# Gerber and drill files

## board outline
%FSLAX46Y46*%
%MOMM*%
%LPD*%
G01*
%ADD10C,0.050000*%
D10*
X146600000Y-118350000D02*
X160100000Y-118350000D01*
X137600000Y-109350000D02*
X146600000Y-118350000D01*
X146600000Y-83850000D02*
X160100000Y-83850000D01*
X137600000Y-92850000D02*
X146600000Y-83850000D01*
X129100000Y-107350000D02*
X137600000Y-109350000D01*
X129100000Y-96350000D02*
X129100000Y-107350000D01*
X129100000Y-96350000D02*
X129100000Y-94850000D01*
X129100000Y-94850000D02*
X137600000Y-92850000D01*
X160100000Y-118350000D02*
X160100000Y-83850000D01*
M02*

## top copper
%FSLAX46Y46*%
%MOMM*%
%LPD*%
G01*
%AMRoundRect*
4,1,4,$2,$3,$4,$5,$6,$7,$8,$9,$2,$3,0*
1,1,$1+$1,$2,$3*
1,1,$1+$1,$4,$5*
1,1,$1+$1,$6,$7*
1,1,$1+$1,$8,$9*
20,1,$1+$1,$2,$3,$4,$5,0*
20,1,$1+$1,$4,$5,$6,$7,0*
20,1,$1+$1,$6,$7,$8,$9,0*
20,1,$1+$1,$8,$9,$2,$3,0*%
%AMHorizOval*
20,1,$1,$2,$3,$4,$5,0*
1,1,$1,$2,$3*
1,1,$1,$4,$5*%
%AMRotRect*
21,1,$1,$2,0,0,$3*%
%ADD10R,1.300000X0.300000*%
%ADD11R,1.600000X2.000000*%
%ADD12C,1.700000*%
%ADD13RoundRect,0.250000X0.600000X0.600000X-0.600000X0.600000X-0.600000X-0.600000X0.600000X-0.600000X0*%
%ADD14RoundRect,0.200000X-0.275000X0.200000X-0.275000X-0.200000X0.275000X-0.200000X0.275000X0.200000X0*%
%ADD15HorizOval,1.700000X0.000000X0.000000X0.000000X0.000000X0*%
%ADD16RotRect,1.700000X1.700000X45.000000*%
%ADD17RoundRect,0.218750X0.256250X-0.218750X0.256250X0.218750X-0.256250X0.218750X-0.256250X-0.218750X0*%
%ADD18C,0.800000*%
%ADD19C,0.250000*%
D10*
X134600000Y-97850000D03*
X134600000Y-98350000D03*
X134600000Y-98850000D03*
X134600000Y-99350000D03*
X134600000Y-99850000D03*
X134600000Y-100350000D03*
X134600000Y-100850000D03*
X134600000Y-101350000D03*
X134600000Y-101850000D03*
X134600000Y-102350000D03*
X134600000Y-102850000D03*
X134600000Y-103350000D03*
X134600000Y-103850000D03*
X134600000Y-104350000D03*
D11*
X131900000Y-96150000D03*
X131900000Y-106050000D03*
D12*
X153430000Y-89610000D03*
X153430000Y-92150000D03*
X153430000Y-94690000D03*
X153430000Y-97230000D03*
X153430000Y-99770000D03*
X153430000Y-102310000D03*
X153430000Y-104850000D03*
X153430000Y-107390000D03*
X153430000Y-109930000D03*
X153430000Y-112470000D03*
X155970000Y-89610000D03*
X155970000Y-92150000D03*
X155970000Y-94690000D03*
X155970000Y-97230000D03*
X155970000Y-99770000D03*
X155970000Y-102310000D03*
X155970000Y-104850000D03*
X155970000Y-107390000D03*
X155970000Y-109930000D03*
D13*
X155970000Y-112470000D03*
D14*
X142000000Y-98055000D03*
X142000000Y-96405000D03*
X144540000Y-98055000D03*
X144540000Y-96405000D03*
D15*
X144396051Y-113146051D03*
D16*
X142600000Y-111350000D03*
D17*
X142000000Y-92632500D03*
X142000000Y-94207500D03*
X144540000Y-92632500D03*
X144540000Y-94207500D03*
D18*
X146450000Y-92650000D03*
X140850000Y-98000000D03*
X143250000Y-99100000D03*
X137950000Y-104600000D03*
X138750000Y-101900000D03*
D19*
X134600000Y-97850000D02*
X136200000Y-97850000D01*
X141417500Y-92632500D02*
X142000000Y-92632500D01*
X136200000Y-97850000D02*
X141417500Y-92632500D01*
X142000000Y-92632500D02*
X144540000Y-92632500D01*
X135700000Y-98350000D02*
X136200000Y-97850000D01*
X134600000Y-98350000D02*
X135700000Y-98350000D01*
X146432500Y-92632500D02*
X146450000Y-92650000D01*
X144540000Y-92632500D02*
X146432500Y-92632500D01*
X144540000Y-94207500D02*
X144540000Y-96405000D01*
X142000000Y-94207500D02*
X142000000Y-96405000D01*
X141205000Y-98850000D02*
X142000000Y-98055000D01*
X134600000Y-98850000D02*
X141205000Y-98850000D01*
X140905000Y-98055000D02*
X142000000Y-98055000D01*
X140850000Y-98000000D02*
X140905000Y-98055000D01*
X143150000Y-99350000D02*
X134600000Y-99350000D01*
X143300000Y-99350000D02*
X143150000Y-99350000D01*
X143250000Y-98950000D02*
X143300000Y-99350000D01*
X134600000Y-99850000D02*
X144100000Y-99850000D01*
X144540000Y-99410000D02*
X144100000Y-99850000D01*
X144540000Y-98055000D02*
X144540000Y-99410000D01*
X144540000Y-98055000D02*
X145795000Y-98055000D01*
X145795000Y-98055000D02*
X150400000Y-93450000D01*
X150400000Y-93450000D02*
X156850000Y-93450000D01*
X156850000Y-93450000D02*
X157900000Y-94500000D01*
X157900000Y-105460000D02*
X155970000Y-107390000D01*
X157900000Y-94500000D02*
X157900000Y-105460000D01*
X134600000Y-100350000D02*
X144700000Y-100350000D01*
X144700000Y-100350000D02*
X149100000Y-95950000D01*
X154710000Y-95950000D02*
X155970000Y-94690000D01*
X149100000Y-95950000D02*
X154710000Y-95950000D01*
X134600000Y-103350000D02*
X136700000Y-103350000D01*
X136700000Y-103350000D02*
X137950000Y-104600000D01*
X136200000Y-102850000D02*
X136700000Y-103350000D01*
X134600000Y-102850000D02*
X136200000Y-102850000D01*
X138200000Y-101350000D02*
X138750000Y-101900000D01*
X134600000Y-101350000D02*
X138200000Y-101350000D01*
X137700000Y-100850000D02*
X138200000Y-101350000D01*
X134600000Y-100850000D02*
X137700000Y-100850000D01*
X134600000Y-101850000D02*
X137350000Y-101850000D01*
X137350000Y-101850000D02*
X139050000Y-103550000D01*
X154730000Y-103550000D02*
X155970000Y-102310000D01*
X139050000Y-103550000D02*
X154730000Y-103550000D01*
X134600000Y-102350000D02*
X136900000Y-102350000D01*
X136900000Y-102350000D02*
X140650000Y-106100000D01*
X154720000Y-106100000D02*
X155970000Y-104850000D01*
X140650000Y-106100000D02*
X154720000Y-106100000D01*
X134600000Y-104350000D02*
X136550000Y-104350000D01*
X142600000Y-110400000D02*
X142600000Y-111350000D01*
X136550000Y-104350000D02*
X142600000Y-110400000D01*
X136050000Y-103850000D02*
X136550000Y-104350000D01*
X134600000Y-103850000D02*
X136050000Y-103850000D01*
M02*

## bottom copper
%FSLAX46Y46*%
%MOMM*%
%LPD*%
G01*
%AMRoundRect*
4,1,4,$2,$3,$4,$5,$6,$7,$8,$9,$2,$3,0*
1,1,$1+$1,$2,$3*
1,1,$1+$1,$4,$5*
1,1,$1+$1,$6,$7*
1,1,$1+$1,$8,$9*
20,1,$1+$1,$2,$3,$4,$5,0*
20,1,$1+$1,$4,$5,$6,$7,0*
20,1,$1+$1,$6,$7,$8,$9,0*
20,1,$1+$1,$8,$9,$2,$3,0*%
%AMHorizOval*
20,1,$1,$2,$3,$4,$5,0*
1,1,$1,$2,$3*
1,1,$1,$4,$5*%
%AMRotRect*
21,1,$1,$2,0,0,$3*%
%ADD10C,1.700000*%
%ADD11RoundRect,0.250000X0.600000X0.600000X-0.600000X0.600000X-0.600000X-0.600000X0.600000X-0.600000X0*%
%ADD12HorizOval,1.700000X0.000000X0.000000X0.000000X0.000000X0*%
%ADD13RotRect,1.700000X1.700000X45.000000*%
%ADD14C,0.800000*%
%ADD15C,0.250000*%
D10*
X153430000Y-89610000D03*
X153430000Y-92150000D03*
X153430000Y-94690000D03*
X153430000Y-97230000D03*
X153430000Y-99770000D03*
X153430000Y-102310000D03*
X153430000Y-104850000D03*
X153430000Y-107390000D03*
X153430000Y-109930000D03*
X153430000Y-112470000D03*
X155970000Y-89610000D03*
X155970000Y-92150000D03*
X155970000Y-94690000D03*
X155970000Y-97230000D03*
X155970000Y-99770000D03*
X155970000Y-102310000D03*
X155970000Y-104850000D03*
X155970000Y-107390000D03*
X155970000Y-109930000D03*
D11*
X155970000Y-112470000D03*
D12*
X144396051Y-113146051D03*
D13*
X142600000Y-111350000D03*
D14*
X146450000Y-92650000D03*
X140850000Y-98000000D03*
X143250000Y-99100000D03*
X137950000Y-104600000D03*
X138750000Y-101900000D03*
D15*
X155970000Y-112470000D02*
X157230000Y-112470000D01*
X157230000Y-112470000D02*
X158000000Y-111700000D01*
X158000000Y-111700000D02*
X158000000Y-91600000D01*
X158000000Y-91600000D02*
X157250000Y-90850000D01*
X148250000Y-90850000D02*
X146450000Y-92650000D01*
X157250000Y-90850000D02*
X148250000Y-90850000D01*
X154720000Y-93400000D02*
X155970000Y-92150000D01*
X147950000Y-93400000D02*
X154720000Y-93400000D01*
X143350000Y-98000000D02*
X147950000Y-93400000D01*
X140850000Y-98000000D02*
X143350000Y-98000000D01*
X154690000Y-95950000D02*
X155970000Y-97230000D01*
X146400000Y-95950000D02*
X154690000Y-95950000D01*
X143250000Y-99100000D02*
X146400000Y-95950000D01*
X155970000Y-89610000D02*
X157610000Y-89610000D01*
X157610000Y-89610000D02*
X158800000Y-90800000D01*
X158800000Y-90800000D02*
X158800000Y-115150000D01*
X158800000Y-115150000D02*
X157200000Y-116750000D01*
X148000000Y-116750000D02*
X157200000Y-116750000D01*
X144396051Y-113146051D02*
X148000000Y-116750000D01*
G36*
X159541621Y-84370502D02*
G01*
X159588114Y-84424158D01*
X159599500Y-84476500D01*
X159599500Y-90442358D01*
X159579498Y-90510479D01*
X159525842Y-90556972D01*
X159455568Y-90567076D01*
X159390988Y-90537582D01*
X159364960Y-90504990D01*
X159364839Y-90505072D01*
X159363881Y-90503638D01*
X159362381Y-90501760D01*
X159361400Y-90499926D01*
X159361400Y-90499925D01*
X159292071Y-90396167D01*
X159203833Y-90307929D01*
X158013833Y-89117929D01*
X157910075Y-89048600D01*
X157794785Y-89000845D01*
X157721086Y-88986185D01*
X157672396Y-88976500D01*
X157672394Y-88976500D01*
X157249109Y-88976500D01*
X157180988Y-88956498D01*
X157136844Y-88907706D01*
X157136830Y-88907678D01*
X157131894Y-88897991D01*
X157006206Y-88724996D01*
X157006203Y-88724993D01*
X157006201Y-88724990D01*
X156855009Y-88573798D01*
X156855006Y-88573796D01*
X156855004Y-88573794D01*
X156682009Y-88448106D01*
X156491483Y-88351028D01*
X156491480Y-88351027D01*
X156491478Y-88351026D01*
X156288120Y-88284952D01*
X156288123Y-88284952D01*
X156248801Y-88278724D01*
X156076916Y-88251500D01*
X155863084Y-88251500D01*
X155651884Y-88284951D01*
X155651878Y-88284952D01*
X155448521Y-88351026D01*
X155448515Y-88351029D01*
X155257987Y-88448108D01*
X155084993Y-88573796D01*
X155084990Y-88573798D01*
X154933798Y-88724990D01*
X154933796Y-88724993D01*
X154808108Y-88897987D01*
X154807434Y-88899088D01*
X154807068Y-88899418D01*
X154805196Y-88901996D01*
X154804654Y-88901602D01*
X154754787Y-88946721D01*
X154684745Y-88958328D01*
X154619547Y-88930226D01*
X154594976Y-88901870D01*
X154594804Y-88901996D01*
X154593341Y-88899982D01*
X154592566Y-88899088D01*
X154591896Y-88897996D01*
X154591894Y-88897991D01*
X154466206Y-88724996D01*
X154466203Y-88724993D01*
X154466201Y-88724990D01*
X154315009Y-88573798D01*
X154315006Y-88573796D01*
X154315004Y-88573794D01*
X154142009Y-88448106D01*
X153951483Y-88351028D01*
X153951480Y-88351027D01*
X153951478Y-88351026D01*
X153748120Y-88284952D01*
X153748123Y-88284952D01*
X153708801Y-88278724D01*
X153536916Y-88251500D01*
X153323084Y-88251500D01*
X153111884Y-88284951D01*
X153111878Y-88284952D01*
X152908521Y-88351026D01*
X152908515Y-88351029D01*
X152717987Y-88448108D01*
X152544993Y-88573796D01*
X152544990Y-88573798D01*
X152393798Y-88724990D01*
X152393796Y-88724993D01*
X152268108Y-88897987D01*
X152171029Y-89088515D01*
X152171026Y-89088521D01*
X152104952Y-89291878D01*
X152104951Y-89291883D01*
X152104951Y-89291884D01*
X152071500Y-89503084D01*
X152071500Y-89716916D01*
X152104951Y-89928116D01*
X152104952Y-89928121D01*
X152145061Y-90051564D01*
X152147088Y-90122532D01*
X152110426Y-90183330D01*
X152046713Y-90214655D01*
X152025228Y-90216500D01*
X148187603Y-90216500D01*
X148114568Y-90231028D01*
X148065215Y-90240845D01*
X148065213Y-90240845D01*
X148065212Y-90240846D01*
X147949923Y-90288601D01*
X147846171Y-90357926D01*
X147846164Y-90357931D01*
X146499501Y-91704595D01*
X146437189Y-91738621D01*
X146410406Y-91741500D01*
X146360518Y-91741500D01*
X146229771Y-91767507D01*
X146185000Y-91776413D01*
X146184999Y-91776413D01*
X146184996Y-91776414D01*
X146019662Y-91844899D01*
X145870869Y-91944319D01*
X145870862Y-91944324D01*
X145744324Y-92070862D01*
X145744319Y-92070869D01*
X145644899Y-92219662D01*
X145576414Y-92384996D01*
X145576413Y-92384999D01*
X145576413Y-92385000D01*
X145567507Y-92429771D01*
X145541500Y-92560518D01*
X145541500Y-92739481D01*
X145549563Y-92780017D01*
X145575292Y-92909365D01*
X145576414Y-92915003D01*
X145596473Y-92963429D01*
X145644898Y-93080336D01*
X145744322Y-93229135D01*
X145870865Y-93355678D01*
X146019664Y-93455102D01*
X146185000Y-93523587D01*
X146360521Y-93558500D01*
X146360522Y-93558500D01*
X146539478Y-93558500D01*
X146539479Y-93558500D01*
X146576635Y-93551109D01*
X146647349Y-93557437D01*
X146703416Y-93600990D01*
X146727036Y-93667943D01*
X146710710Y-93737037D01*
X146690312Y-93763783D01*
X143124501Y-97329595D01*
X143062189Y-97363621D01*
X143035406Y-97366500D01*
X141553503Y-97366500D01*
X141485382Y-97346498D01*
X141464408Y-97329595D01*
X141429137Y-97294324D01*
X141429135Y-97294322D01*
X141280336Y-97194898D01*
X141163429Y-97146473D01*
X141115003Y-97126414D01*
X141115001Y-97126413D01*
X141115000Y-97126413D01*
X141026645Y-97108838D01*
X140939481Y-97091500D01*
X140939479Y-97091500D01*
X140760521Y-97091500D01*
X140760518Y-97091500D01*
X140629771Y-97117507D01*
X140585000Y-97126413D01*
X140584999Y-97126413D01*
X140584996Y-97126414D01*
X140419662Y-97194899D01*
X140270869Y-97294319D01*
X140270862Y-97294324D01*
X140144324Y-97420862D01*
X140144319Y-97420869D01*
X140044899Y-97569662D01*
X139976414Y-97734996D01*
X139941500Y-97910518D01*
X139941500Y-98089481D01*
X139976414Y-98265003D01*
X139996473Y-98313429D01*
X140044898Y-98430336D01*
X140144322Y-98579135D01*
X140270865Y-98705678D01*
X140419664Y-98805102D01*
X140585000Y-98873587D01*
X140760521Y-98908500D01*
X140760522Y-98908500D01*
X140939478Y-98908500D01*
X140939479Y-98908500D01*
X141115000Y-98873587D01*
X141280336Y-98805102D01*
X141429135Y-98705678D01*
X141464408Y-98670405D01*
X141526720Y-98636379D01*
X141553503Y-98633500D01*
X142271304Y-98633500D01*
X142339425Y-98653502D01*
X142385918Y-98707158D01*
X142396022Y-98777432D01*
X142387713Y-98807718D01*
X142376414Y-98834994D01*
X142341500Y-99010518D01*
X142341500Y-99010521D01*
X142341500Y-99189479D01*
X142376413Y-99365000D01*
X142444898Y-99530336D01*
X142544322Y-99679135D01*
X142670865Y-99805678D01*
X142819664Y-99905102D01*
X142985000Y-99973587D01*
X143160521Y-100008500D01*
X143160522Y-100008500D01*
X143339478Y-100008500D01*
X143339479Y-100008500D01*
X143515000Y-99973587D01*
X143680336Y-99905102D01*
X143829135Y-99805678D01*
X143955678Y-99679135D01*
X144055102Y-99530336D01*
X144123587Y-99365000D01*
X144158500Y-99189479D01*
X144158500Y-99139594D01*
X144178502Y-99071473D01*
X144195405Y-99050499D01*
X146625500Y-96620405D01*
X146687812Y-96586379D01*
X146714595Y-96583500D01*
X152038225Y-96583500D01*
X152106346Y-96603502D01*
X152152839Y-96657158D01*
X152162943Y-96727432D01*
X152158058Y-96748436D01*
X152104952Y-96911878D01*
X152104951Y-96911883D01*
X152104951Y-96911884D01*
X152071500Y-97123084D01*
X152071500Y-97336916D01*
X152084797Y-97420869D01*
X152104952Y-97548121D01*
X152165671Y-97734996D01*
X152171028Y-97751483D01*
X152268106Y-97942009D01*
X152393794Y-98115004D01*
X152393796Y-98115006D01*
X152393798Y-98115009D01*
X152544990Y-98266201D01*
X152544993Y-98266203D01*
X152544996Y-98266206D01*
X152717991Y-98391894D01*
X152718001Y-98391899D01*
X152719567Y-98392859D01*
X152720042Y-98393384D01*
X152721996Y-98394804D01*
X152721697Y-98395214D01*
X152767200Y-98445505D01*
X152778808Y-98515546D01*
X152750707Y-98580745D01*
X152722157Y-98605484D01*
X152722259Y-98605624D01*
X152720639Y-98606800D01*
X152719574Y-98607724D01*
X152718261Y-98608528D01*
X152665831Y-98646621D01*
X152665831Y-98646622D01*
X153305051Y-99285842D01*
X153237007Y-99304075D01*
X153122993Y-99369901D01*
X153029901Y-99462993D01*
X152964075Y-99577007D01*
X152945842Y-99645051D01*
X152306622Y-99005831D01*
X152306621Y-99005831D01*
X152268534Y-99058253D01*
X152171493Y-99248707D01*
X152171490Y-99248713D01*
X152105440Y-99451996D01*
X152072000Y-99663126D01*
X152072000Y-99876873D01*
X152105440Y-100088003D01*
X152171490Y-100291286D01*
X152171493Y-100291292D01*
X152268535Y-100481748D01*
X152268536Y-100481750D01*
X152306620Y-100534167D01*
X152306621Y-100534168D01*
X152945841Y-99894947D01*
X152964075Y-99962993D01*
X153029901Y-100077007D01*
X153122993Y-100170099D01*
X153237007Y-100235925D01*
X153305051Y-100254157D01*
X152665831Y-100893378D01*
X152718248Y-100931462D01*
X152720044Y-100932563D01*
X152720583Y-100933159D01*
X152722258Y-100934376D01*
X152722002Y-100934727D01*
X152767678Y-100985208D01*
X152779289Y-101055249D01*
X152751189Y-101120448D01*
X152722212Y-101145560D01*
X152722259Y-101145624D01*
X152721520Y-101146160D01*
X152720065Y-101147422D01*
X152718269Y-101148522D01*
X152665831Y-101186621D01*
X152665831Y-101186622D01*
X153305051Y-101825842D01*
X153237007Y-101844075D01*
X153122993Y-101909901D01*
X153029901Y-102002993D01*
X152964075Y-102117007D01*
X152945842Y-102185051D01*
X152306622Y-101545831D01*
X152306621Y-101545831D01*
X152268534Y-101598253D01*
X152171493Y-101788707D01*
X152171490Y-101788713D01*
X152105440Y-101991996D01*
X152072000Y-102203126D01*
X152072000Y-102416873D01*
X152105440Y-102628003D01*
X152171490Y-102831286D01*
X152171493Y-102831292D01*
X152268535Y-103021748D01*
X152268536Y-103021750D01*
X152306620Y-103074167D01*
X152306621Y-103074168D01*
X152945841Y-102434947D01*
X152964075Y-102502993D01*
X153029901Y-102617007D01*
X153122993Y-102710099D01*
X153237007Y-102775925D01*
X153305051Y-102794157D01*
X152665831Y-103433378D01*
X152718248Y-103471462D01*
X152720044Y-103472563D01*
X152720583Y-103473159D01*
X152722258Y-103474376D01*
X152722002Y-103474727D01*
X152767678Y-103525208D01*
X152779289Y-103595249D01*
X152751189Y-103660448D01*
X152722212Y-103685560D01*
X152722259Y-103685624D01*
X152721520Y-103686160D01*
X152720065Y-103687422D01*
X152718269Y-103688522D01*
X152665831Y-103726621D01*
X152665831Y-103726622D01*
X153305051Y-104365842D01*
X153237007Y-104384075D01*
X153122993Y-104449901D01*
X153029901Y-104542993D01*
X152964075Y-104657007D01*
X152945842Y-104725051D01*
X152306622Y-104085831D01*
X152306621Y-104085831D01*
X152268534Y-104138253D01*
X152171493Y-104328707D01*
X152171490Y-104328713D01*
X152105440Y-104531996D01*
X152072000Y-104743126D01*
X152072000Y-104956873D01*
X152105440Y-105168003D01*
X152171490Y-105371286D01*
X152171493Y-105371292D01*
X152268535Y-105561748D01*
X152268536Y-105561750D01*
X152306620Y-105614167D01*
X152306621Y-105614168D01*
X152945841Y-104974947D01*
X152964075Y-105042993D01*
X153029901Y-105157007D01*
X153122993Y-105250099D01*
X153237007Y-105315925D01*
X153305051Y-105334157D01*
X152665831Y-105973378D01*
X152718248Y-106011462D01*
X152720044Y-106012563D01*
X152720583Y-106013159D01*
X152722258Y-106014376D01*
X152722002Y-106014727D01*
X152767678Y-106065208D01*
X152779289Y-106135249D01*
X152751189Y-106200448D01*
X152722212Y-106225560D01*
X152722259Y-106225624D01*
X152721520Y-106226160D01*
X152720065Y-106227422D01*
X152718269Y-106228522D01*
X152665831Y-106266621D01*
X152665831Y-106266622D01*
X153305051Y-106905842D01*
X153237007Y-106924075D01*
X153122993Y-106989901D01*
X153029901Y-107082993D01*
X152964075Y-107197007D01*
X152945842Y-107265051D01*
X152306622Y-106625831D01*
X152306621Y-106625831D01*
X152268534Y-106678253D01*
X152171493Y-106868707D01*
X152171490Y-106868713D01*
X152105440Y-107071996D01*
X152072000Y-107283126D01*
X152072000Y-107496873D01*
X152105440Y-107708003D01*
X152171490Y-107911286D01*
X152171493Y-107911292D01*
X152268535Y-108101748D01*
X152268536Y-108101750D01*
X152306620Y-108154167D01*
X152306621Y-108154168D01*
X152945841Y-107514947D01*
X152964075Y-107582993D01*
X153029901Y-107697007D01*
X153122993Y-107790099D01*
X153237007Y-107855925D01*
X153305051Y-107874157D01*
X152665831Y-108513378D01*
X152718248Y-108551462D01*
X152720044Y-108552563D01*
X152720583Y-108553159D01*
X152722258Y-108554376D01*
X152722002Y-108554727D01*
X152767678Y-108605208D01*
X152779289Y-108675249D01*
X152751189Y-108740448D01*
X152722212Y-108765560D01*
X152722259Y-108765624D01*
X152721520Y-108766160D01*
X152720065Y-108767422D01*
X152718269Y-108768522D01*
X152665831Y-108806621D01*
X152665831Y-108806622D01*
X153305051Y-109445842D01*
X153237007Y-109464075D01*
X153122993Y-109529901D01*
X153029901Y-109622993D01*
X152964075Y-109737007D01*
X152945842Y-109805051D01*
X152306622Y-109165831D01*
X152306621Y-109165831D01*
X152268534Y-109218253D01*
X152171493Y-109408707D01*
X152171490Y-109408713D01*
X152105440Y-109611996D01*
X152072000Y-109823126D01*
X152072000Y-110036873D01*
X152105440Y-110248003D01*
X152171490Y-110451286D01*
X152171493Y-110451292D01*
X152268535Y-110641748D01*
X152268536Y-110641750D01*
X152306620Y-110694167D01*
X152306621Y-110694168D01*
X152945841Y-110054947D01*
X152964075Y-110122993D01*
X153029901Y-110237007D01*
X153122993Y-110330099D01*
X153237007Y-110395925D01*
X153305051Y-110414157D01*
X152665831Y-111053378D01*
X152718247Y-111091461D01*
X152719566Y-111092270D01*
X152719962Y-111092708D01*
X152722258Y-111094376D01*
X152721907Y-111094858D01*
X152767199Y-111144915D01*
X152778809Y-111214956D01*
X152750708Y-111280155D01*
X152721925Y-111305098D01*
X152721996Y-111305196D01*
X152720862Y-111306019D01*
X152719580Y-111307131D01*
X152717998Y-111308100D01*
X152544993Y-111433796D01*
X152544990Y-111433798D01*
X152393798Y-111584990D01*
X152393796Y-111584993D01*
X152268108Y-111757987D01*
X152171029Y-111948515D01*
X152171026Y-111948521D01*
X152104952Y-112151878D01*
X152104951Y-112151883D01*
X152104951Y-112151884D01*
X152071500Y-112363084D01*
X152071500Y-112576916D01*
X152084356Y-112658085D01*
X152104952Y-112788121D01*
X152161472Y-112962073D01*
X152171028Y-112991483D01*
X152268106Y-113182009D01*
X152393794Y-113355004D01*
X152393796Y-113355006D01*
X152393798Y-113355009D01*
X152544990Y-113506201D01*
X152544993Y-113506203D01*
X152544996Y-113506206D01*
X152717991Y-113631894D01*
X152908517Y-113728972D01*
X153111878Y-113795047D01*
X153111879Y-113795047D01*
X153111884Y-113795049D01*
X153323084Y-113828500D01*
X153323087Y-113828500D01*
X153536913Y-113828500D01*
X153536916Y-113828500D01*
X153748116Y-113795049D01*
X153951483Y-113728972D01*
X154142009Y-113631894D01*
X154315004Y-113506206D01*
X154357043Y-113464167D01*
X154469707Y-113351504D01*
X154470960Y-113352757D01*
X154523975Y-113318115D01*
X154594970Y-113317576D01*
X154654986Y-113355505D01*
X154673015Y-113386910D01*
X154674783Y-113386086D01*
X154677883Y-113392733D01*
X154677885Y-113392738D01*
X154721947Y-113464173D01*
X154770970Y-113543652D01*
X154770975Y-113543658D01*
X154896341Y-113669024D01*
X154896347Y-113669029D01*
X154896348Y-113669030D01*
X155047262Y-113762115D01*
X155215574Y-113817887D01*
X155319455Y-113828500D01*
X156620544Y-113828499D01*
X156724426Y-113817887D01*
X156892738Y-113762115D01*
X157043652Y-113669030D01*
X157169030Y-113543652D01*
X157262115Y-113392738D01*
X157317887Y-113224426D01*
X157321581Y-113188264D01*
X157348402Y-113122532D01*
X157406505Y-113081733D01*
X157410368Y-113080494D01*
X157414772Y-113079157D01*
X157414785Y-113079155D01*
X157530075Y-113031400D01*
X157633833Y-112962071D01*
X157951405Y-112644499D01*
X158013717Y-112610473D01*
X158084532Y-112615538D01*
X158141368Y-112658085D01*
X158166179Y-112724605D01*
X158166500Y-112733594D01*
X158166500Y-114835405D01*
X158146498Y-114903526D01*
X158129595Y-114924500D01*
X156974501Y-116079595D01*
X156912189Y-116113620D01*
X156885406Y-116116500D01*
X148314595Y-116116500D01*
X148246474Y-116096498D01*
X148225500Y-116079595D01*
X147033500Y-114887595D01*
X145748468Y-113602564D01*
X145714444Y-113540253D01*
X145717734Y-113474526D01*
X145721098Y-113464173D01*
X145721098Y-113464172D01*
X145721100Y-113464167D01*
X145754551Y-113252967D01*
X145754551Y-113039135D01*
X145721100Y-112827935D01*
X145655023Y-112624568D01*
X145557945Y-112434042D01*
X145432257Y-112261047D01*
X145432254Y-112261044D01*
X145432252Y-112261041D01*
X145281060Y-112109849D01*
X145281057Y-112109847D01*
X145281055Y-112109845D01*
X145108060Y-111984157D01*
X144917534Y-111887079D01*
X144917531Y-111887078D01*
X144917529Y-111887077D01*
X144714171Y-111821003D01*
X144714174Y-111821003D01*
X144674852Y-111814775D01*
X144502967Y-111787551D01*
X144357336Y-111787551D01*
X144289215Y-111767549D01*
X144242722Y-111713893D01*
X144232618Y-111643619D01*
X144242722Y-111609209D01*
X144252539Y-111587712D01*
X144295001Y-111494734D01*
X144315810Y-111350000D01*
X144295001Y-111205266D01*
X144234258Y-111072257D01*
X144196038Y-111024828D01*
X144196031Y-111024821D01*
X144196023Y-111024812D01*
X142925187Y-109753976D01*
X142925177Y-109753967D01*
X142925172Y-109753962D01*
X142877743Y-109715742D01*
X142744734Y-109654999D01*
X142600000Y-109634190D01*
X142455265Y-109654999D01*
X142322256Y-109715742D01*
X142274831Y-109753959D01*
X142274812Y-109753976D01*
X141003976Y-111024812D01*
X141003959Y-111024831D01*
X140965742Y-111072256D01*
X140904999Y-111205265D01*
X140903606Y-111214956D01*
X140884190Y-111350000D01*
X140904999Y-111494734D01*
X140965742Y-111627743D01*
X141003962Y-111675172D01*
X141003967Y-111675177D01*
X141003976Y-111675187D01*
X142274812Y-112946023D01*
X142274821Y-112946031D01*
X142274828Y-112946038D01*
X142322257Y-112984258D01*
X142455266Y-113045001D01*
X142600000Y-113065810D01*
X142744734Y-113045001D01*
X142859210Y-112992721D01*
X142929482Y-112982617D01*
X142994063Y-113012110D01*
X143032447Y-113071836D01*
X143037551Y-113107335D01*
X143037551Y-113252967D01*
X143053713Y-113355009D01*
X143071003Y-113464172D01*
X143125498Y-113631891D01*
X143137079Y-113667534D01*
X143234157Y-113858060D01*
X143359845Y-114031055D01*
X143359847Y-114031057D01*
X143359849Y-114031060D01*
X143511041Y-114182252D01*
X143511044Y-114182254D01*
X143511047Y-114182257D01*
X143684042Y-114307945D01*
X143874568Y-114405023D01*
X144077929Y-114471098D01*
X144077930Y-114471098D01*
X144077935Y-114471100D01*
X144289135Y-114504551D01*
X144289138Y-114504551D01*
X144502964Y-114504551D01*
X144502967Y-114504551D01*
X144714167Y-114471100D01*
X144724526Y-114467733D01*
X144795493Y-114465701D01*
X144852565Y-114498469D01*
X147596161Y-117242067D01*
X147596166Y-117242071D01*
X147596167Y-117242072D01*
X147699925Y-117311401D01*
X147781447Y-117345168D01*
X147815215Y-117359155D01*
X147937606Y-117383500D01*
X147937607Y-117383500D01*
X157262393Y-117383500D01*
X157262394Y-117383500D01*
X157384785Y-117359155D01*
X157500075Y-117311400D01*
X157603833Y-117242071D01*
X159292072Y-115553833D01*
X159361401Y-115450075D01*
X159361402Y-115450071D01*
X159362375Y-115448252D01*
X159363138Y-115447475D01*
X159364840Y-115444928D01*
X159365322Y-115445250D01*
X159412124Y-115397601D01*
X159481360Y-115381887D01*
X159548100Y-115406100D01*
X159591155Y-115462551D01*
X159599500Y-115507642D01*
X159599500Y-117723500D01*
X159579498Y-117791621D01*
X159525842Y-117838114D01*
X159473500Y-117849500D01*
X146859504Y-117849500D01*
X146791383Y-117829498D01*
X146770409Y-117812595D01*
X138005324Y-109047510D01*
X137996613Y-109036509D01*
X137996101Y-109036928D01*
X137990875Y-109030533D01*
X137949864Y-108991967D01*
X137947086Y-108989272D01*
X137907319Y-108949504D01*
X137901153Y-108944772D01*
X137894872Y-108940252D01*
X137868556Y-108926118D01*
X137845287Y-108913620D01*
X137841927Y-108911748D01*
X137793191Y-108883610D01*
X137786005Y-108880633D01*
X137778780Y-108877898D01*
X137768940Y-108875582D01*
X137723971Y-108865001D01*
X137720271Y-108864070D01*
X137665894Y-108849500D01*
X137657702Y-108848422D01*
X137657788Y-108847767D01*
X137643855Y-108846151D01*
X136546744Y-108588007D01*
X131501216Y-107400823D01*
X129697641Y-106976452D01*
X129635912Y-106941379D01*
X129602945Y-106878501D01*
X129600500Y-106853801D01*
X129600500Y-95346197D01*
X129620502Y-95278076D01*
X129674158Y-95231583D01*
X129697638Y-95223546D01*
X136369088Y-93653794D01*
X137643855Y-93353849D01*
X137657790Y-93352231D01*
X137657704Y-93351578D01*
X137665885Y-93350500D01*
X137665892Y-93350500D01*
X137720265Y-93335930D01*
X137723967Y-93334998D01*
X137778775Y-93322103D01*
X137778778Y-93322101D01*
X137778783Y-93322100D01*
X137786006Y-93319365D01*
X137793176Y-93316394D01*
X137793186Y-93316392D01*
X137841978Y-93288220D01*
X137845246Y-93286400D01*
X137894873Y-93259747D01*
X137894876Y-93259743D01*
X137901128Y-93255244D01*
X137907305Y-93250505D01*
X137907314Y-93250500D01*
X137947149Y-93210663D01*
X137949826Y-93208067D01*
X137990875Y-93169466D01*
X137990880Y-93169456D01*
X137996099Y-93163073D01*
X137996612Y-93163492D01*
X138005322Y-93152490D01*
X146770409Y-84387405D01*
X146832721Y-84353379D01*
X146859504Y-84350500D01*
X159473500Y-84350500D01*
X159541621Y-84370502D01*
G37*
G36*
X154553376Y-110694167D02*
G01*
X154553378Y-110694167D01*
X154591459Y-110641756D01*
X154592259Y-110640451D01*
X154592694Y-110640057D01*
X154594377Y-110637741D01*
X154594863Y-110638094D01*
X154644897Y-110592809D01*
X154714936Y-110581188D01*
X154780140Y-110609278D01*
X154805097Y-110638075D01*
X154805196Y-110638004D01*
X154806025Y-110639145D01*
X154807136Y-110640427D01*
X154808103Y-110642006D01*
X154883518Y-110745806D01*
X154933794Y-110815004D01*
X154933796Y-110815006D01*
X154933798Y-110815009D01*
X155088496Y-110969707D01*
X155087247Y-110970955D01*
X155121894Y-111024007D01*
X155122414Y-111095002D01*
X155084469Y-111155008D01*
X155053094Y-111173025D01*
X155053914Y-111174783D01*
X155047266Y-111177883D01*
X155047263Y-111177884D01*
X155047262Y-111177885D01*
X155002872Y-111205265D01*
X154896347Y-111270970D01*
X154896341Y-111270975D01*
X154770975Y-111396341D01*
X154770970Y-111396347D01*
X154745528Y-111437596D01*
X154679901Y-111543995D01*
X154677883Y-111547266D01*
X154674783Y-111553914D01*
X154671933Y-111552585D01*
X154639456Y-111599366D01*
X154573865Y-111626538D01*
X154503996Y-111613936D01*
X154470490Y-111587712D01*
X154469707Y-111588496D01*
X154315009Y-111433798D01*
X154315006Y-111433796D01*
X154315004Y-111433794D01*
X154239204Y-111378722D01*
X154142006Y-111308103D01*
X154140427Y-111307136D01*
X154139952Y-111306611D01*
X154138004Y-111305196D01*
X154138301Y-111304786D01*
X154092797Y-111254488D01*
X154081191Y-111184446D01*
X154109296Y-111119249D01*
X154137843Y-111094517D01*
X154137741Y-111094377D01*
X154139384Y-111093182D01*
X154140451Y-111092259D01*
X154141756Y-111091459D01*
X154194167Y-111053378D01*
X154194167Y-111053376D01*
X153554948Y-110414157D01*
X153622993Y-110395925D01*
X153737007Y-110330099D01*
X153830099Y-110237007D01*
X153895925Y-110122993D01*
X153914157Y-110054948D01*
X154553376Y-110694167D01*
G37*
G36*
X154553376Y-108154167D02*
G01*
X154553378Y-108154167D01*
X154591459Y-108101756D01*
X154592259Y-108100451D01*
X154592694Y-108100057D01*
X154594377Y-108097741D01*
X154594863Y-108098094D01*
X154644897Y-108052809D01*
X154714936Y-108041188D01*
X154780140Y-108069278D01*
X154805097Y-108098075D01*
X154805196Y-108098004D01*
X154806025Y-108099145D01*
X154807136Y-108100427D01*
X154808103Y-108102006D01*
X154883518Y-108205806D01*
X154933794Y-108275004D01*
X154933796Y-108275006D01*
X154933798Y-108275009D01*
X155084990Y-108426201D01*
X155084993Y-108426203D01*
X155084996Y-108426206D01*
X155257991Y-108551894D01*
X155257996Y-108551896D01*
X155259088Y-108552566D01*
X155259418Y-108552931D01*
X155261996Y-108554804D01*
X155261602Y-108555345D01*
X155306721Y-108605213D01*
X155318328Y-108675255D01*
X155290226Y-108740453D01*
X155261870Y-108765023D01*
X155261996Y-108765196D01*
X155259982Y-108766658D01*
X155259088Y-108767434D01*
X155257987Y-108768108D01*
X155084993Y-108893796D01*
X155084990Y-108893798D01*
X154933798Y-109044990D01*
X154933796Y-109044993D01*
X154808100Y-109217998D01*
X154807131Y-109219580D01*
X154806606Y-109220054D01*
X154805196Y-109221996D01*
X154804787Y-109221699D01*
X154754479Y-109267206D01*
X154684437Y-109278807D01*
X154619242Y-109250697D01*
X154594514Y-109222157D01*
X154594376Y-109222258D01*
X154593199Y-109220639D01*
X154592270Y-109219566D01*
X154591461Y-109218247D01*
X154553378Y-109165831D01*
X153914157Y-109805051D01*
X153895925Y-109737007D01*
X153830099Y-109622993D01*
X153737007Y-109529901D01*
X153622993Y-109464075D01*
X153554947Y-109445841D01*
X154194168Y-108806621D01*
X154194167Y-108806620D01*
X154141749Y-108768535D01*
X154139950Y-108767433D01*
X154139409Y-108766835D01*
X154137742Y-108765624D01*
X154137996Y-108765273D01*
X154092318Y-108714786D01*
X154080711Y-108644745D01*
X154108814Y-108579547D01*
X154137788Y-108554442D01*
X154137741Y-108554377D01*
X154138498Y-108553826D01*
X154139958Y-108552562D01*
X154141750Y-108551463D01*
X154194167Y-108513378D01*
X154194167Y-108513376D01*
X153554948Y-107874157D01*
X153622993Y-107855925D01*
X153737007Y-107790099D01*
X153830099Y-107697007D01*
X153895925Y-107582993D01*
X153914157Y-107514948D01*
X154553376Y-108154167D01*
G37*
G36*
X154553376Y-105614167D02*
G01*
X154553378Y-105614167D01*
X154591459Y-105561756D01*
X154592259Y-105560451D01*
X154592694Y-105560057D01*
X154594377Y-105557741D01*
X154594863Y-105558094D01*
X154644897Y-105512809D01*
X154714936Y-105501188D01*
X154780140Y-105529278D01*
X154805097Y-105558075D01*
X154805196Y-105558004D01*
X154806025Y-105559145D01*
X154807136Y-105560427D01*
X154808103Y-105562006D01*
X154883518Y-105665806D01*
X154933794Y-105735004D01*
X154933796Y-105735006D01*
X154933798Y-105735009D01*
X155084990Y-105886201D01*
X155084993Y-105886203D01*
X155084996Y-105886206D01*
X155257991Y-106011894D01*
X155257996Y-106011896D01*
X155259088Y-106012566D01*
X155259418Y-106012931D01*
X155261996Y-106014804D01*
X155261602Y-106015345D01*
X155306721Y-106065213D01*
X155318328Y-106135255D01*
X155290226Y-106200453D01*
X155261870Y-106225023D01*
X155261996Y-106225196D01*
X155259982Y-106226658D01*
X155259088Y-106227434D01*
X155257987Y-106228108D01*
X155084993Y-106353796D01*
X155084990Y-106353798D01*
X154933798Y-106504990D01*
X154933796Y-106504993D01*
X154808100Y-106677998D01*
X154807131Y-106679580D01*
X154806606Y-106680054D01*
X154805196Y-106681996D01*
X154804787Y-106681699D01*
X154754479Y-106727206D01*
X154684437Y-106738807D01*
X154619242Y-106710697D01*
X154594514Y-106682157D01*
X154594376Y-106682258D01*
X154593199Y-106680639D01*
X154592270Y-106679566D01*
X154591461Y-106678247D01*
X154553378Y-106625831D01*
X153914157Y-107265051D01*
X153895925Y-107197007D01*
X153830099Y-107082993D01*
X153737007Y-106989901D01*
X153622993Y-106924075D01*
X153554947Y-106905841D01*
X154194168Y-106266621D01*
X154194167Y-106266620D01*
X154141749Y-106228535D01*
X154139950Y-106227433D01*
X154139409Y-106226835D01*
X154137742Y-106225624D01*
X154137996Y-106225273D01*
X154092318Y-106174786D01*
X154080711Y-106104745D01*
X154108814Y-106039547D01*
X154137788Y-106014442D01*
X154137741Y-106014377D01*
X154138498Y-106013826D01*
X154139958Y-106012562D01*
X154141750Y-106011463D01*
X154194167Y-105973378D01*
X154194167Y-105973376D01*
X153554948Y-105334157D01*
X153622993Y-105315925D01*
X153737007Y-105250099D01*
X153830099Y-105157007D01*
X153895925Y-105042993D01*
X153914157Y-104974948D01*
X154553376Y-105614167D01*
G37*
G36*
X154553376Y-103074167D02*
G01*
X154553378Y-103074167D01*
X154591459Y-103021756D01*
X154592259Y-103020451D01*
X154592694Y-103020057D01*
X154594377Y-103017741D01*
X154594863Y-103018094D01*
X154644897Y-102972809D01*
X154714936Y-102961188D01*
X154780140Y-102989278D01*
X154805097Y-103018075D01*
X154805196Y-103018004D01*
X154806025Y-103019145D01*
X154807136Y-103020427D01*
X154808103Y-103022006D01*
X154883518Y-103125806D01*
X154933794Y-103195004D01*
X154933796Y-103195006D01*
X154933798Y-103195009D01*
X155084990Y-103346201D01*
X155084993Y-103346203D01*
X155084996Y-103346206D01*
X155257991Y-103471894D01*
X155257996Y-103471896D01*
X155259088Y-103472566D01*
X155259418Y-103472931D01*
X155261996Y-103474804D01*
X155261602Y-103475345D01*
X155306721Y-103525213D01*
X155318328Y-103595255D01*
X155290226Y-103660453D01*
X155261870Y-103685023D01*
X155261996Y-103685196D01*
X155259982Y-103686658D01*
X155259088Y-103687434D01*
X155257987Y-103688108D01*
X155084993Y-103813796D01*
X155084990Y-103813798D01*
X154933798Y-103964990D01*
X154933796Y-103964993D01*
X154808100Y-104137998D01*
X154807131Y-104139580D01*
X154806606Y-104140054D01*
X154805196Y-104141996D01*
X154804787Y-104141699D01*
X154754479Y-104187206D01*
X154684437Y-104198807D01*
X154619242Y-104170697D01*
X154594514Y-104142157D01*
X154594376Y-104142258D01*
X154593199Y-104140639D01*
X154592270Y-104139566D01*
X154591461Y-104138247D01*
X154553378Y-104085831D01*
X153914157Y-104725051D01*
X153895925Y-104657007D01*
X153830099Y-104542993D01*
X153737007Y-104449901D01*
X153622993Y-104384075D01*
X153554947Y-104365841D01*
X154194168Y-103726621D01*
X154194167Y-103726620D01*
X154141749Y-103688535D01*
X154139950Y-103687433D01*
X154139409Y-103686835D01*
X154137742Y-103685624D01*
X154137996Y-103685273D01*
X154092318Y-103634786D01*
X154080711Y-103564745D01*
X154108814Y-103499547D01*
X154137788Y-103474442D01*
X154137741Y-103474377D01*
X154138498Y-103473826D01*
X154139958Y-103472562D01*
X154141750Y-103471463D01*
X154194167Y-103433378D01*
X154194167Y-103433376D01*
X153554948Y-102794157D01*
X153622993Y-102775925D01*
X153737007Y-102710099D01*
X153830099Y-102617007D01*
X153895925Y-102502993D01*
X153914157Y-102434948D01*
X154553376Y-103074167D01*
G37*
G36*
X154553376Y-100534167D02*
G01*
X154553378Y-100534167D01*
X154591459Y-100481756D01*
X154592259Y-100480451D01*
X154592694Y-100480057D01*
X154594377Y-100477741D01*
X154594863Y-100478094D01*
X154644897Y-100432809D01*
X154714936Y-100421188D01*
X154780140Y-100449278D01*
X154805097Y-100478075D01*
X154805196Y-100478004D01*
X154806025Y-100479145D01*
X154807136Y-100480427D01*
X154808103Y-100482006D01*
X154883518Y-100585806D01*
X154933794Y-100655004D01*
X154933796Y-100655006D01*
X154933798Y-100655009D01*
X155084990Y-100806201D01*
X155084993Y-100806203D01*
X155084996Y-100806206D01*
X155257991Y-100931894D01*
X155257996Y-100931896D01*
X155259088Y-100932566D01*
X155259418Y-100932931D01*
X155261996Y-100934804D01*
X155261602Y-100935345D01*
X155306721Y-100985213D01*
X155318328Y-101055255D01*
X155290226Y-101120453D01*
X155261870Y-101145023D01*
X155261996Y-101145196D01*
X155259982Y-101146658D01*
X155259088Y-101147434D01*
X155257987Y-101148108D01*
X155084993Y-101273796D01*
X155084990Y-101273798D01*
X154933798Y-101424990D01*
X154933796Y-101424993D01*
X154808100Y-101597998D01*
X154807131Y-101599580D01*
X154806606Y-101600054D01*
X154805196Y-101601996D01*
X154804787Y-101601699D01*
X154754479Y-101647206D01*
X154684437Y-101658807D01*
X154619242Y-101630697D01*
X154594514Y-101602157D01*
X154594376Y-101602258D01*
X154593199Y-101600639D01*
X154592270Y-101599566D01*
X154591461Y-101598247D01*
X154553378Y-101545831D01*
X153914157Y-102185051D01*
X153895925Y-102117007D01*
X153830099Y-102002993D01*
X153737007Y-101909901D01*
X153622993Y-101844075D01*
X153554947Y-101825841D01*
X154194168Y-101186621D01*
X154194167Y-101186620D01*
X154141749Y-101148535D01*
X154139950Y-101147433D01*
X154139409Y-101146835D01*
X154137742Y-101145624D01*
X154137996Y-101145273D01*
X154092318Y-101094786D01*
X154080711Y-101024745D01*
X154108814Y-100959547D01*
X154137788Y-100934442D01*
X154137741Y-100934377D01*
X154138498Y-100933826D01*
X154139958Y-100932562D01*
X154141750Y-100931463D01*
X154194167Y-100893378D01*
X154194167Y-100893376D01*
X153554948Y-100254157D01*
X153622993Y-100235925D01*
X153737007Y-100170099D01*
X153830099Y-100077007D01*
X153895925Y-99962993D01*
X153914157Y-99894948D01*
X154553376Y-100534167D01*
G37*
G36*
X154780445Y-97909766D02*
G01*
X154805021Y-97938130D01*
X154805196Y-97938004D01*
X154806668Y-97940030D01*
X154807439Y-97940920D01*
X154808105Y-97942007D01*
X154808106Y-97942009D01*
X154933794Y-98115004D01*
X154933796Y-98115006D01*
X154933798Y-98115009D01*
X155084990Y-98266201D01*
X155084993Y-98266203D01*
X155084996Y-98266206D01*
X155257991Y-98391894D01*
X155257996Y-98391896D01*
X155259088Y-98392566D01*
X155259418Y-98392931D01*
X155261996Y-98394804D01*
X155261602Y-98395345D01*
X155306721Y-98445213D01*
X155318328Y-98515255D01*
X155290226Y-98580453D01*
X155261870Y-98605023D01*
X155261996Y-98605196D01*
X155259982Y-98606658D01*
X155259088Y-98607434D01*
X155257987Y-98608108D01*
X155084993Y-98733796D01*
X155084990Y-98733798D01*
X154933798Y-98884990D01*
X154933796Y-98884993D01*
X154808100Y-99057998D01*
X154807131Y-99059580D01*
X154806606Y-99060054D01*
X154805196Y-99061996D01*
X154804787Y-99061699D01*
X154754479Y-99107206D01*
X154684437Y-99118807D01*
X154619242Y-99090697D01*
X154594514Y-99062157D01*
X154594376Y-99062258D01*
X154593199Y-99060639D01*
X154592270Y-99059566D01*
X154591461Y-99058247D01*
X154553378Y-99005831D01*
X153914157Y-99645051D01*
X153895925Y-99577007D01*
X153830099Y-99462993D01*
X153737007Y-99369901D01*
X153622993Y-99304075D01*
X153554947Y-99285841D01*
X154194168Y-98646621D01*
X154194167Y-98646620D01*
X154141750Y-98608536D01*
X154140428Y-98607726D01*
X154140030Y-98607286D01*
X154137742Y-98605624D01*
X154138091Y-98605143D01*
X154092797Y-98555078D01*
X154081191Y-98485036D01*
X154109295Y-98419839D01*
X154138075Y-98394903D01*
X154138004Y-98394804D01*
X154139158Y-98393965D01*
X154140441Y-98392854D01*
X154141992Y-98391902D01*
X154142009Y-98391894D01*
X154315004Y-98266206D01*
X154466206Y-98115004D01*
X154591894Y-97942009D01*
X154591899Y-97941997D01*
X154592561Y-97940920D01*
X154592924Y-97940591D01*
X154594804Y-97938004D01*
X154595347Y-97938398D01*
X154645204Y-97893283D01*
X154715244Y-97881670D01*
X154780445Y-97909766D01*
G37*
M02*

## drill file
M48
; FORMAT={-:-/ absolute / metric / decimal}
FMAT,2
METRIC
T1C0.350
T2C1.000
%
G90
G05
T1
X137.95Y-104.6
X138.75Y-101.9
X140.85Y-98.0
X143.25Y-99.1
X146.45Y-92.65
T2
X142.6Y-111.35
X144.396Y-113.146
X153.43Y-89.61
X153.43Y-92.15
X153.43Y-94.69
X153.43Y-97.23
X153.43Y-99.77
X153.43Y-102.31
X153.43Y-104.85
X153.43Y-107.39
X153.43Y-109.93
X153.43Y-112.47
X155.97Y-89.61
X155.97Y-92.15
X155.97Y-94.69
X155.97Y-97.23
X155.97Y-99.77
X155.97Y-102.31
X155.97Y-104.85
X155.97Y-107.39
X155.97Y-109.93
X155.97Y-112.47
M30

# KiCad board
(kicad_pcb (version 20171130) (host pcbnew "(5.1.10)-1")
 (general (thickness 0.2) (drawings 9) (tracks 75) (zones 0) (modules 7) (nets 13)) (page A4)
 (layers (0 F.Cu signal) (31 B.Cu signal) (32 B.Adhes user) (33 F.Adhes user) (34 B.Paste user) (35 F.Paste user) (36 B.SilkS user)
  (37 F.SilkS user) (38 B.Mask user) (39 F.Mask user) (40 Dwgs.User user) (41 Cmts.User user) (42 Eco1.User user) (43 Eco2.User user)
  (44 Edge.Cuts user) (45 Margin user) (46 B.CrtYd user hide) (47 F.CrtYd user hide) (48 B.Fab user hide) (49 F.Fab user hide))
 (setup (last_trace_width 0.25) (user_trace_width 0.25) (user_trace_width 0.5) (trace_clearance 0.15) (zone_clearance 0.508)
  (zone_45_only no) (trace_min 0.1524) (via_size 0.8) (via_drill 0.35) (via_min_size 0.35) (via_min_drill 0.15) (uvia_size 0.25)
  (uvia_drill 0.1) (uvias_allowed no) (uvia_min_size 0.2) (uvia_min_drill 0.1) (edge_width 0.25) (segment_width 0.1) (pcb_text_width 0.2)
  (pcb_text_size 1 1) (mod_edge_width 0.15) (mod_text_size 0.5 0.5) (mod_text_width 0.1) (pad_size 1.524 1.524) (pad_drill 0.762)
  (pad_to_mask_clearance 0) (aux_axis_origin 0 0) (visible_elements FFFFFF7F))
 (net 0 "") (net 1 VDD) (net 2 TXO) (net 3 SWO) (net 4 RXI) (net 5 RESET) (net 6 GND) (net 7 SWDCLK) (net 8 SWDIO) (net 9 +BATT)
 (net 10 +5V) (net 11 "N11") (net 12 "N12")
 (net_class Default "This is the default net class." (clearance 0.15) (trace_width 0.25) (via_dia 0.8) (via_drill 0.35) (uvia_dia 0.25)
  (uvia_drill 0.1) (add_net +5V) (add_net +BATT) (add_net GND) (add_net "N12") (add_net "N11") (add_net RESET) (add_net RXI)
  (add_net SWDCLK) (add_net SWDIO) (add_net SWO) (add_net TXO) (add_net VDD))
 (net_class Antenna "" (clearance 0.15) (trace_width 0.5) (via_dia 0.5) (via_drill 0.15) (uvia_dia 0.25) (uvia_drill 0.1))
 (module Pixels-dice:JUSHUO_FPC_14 (layer F.Cu) (at 133.25 101.1 270)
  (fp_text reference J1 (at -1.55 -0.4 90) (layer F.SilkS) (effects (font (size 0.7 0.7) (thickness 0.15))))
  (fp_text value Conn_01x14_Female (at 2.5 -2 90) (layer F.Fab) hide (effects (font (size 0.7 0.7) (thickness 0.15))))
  (pad 1 smd rect (at -3.25 -1.35 270) (size 0.3 1.3) (layers F.Cu F.Paste F.Mask) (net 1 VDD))
  (pad 2 smd rect (at -2.75 -1.35 270) (size 0.3 1.3) (layers F.Cu F.Paste F.Mask) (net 1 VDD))
  (pad 3 smd rect (at -2.25 -1.35 270) (size 0.3 1.3) (layers F.Cu F.Paste F.Mask) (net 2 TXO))
  (pad 4 smd rect (at -1.75 -1.35 270) (size 0.3 1.3) (layers F.Cu F.Paste F.Mask) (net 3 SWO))
  (pad 5 smd rect (at -1.25 -1.35 270) (size 0.3 1.3) (layers F.Cu F.Paste F.Mask) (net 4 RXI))
  (pad 6 smd rect (at -0.75 -1.35 270) (size 0.3 1.3) (layers F.Cu F.Paste F.Mask) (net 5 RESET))
  (pad 7 smd rect (at -0.25 -1.35 270) (size 0.3 1.3) (layers F.Cu F.Paste F.Mask) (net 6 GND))
  (pad 8 smd rect (at 0.25 -1.35 270) (size 0.3 1.3) (layers F.Cu F.Paste F.Mask) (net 6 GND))
  (pad 9 smd rect (at 0.75 -1.35 270) (size 0.3 1.3) (layers F.Cu F.Paste F.Mask) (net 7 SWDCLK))
  (pad 10 smd rect (at 1.25 -1.35 270) (size 0.3 1.3) (layers F.Cu F.Paste F.Mask) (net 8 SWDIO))
  (pad 11 smd rect (at 1.75 -1.35 270) (size 0.3 1.3) (layers F.Cu F.Paste F.Mask) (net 6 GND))
  (pad 12 smd rect (at 2.25 -1.35 270) (size 0.3 1.3) (layers F.Cu F.Paste F.Mask) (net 6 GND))
  (pad 13 smd rect (at 2.75 -1.35 270) (size 0.3 1.3) (layers F.Cu F.Paste F.Mask) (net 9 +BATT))
  (pad 14 smd rect (at 3.25 -1.35 270) (size 0.3 1.3) (layers F.Cu F.Paste F.Mask) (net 9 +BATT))
  (pad 15 smd rect (at -4.95 1.35 270) (size 2 1.6) (layers F.Cu F.Paste F.Mask))
  (pad 16 smd rect (at 4.95 1.35 270) (size 2 1.6) (layers F.Cu F.Paste F.Mask)))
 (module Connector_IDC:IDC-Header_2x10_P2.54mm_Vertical (layer F.Cu) (at 155.97 112.47 180)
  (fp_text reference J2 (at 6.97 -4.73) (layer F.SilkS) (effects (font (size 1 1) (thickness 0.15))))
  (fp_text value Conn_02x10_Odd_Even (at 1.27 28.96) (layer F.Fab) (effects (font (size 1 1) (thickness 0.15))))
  (pad 20 thru_hole circle (at 2.54 22.86 180) (size 1.7 1.7) (drill 1) (layers *.Cu *.Mask))
  (pad 18 thru_hole circle (at 2.54 20.32 180) (size 1.7 1.7) (drill 1) (layers *.Cu *.Mask))
  (pad 16 thru_hole circle (at 2.54 17.78 180) (size 1.7 1.7) (drill 1) (layers *.Cu *.Mask))
  (pad 14 thru_hole circle (at 2.54 15.24 180) (size 1.7 1.7) (drill 1) (layers *.Cu *.Mask))
  (pad 12 thru_hole circle (at 2.54 12.7 180) (size 1.7 1.7) (drill 1) (layers *.Cu *.Mask) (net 6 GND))
  (pad 10 thru_hole circle (at 2.54 10.16 180) (size 1.7 1.7) (drill 1) (layers *.Cu *.Mask) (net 6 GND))
  (pad 8 thru_hole circle (at 2.54 7.62 180) (size 1.7 1.7) (drill 1) (layers *.Cu *.Mask) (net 6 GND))
  (pad 6 thru_hole circle (at 2.54 5.08 180) (size 1.7 1.7) (drill 1) (layers *.Cu *.Mask) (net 6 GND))
  (pad 4 thru_hole circle (at 2.54 2.54 180) (size 1.7 1.7) (drill 1) (layers *.Cu *.Mask) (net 6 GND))
  (pad 2 thru_hole circle (at 2.54 0 180) (size 1.7 1.7) (drill 1) (layers *.Cu *.Mask))
  (pad 19 thru_hole circle (at 0 22.86 180) (size 1.7 1.7) (drill 1) (layers *.Cu *.Mask) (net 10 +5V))
  (pad 17 thru_hole circle (at 0 20.32 180) (size 1.7 1.7) (drill 1) (layers *.Cu *.Mask) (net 2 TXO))
  (pad 15 thru_hole circle (at 0 17.78 180) (size 1.7 1.7) (drill 1) (layers *.Cu *.Mask) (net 5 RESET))
  (pad 13 thru_hole circle (at 0 15.24 180) (size 1.7 1.7) (drill 1) (layers *.Cu *.Mask) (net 3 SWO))
  (pad 11 thru_hole circle (at 0 12.7 180) (size 1.7 1.7) (drill 1) (layers *.Cu *.Mask))
  (pad 9 thru_hole circle (at 0 10.16 180) (size 1.7 1.7) (drill 1) (layers *.Cu *.Mask) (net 7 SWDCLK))
  (pad 7 thru_hole circle (at 0 7.62 180) (size 1.7 1.7) (drill 1) (layers *.Cu *.Mask) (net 8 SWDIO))
  (pad 5 thru_hole circle (at 0 5.08 180) (size 1.7 1.7) (drill 1) (layers *.Cu *.Mask) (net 4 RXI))
  (pad 3 thru_hole circle (at 0 2.54 180) (size 1.7 1.7) (drill 1) (layers *.Cu *.Mask))
  (pad 1 thru_hole roundrect (at 0 0 180) (size 1.7 1.7) (drill 1) (layers *.Cu *.Mask) (roundrect_rratio 0.1470588235294118) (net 1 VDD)))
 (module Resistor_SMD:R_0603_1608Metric (layer F.Cu) (at 142 97.23 270)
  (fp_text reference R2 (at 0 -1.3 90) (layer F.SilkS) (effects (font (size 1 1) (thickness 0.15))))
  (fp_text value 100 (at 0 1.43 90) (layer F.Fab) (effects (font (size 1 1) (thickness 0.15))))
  (pad 2 smd roundrect (at 0.825 0 270) (size 0.8 0.95) (layers F.Cu F.Paste F.Mask) (roundrect_rratio 0.25) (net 2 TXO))
  (pad 1 smd roundrect (at -0.825 0 270) (size 0.8 0.95) (layers F.Cu F.Paste F.Mask) (roundrect_rratio 0.25) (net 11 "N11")))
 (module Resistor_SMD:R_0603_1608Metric (layer F.Cu) (at 144.54 97.23 270)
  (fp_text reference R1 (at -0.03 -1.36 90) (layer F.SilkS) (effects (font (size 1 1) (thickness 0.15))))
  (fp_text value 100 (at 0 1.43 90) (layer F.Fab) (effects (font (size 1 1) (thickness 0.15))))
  (pad 2 smd roundrect (at 0.825 0 270) (size 0.8 0.95) (layers F.Cu F.Paste F.Mask) (roundrect_rratio 0.25) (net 4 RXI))
  (pad 1 smd roundrect (at -0.825 0 270) (size 0.8 0.95) (layers F.Cu F.Paste F.Mask) (roundrect_rratio 0.25) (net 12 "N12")))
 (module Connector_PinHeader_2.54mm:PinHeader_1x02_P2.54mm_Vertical (layer F.Cu) (at 142.6 111.35 45)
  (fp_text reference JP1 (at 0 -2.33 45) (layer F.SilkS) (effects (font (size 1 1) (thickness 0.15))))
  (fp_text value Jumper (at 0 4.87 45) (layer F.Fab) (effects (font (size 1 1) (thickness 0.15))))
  (pad 2 thru_hole oval (at 0 2.54 45) (size 1.7 1.7) (drill 1) (layers *.Cu *.Mask) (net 10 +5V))
  (pad 1 thru_hole rect (at 0 0 45) (size 1.7 1.7) (drill 1) (layers *.Cu *.Mask) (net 9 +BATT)))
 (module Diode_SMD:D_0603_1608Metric (layer F.Cu) (at 142 93.42 90)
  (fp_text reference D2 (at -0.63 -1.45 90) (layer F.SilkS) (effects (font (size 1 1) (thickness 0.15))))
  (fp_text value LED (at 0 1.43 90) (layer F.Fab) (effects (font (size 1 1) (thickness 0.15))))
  (pad 2 smd roundrect (at 0.7875 0 90) (size 0.875 0.95) (layers F.Cu F.Paste F.Mask) (roundrect_rratio 0.25) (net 1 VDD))
  (pad 1 smd roundrect (at -0.7875 0 90) (size 0.875 0.95) (layers F.Cu F.Paste F.Mask) (roundrect_rratio 0.25) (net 11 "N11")))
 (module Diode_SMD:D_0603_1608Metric (layer F.Cu) (at 144.54 93.42 90)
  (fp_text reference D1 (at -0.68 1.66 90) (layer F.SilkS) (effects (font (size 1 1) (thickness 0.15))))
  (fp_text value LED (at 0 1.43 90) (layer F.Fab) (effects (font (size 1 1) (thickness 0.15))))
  (pad 2 smd roundrect (at 0.7875 0 90) (size 0.875 0.95) (layers F.Cu F.Paste F.Mask) (roundrect_rratio 0.25) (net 1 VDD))
  (pad 1 smd roundrect (at -0.7875 0 90) (size 0.875 0.95) (layers F.Cu F.Paste F.Mask) (roundrect_rratio 0.25) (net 12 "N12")))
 (gr_line (start 146.6 118.35) (end 160.1 118.35) (layer Edge.Cuts) (width 0.05))
 (gr_line (start 137.6 109.35) (end 146.6 118.35) (layer Edge.Cuts) (width 0.05))
 (gr_line (start 146.6 83.85) (end 160.1 83.85) (layer Edge.Cuts) (width 0.05))
 (gr_line (start 137.6 92.85) (end 146.6 83.85) (layer Edge.Cuts) (width 0.05))
 (gr_line (start 129.1 107.35) (end 137.6 109.35) (layer Edge.Cuts) (width 0.05))
 (gr_line (start 129.1 96.35) (end 129.1 107.35) (layer Edge.Cuts) (width 0.05))
 (gr_line (start 129.1 96.35) (end 129.1 94.85) (layer Edge.Cuts) (width 0.05))
 (gr_line (start 129.1 94.85) (end 137.6 92.85) (layer Edge.Cuts) (width 0.05))
 (gr_line (start 160.1 118.35) (end 160.1 83.85) (layer Edge.Cuts) (width 0.05))
 (segment (start 134.6 97.85) (end 136.2 97.85) (width 0.25) (layer F.Cu) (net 1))
 (segment (start 141.4175 92.6325) (end 142 92.6325) (width 0.25) (layer F.Cu) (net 1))
 (segment (start 136.2 97.85) (end 141.4175 92.6325) (width 0.25) (layer F.Cu) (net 1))
 (segment (start 142 92.6325) (end 144.54 92.6325) (width 0.25) (layer F.Cu) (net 1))
 (segment (start 135.7 98.35) (end 136.2 97.85) (width 0.25) (layer F.Cu) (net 1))
 (segment (start 134.6 98.35) (end 135.7 98.35) (width 0.25) (layer F.Cu) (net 1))
 (segment (start 155.97 112.47) (end 157.23 112.47) (width 0.25) (layer B.Cu) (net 1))
 (segment (start 157.23 112.47) (end 158 111.7) (width 0.25) (layer B.Cu) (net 1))
 (segment (start 158 111.7) (end 158 91.6) (width 0.25) (layer B.Cu) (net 1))
 (segment (start 158 91.6) (end 157.25 90.85) (width 0.25) (layer B.Cu) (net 1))
 (via (at 146.45 92.65) (size 0.8) (drill 0.35) (layers F.Cu B.Cu) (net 1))
 (segment (start 148.25 90.85) (end 146.45 92.65) (width 0.25) (layer B.Cu) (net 1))
 (segment (start 157.25 90.85) (end 148.25 90.85) (width 0.25) (layer B.Cu) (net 1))
 (segment (start 146.4325 92.6325) (end 146.45 92.65) (width 0.25) (layer F.Cu) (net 1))
 (segment (start 144.54 92.6325) (end 146.4325 92.6325) (width 0.25) (layer F.Cu) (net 1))
 (segment (start 144.54 94.2075) (end 144.54 96.405) (width 0.25) (layer F.Cu) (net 12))
 (segment (start 142 94.2075) (end 142 96.405) (width 0.25) (layer F.Cu) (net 11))
 (segment (start 141.205 98.85) (end 142 98.055) (width 0.25) (layer F.Cu) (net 2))
 (segment (start 134.6 98.85) (end 141.205 98.85) (width 0.25) (layer F.Cu) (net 2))
 (via (at 140.85 98) (size 0.8) (drill 0.35) (layers F.Cu B.Cu) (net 2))
 (segment (start 140.905 98.055) (end 142 98.055) (width 0.25) (layer F.Cu) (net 2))
 (segment (start 140.85 98) (end 140.905 98.055) (width 0.25) (layer F.Cu) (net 2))
 (segment (start 154.72 93.4) (end 155.97 92.15) (width 0.25) (layer B.Cu) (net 2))
 (segment (start 147.95 93.4) (end 154.72 93.4) (width 0.25) (layer B.Cu) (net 2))
 (segment (start 143.35 98) (end 147.95 93.4) (width 0.25) (layer B.Cu) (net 2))
 (segment (start 140.85 98) (end 143.35 98) (width 0.25) (layer B.Cu) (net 2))
 (segment (start 143.15 99.35) (end 134.6 99.35) (width 0.25) (layer F.Cu) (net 3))
 (segment (start 143.3 99.35) (end 143.15 99.35) (width 0.25) (layer F.Cu) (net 3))
 (segment (start 143.25 98.95) (end 143.3 99.35) (width 0.25) (layer F.Cu) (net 3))
 (via (at 143.25 99.1) (size 0.8) (drill 0.35) (layers F.Cu B.Cu) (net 3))
 (segment (start 154.69 95.95) (end 155.97 97.23) (width 0.25) (layer B.Cu) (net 3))
 (segment (start 146.4 95.95) (end 154.69 95.95) (width 0.25) (layer B.Cu) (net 3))
 (segment (start 143.25 99.1) (end 146.4 95.95) (width 0.25) (layer B.Cu) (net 3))
 (segment (start 134.6 99.85) (end 144.1 99.85) (width 0.25) (layer F.Cu) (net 4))
 (segment (start 144.54 99.41) (end 144.1 99.85) (width 0.25) (layer F.Cu) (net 4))
 (segment (start 144.54 98.055) (end 144.54 99.41) (width 0.25) (layer F.Cu) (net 4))
 (segment (start 144.54 98.055) (end 145.795 98.055) (width 0.25) (layer F.Cu) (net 4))
 (segment (start 145.795 98.055) (end 150.4 93.45) (width 0.25) (layer F.Cu) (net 4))
 (segment (start 150.4 93.45) (end 156.85 93.45) (width 0.25) (layer F.Cu) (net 4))
 (segment (start 156.85 93.45) (end 157.9 94.5) (width 0.25) (layer F.Cu) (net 4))
 (segment (start 157.9 105.46) (end 155.97 107.39) (width 0.25) (layer F.Cu) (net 4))
 (segment (start 157.9 94.5) (end 157.9 105.46) (width 0.25) (layer F.Cu) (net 4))
 (segment (start 134.6 100.35) (end 144.7 100.35) (width 0.25) (layer F.Cu) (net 5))
 (segment (start 144.7 100.35) (end 149.1 95.95) (width 0.25) (layer F.Cu) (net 5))
 (segment (start 154.71 95.95) (end 155.97 94.69) (width 0.25) (layer F.Cu) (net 5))
 (segment (start 149.1 95.95) (end 154.71 95.95) (width 0.25) (layer F.Cu) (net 5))
 (segment (start 134.6 103.35) (end 136.7 103.35) (width 0.25) (layer F.Cu) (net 6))
 (via (at 137.95 104.6) (size 0.8) (drill 0.35) (layers F.Cu B.Cu) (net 6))
 (segment (start 136.7 103.35) (end 137.95 104.6) (width 0.25) (layer F.Cu) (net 6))
 (segment (start 136.2 102.85) (end 136.7 103.35) (width 0.25) (layer F.Cu) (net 6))
 (segment (start 134.6 102.85) (end 136.2 102.85) (width 0.25) (layer F.Cu) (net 6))
 (via (at 138.75 101.9) (size 0.8) (drill 0.35) (layers F.Cu B.Cu) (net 6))
 (segment (start 138.2 101.35) (end 138.75 101.9) (width 0.25) (layer F.Cu) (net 6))
 (segment (start 134.6 101.35) (end 138.2 101.35) (width 0.25) (layer F.Cu) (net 6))
 (segment (start 137.7 100.85) (end 138.2 101.35) (width 0.25) (layer F.Cu) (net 6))
 (segment (start 134.6 100.85) (end 137.7 100.85) (width 0.25) (layer F.Cu) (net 6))
 (segment (start 134.6 101.85) (end 137.35 101.85) (width 0.25) (layer F.Cu) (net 7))
 (segment (start 137.35 101.85) (end 139.05 103.55) (width 0.25) (layer F.Cu) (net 7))
 (segment (start 154.73 103.55) (end 155.97 102.31) (width 0.25) (layer F.Cu) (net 7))
 (segment (start 139.05 103.55) (end 154.73 103.55) (width 0.25) (layer F.Cu) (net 7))
 (segment (start 134.6 102.35) (end 136.9 102.35) (width 0.25) (layer F.Cu) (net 8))
 (segment (start 136.9 102.35) (end 140.65 106.1) (width 0.25) (layer F.Cu) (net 8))
 (segment (start 154.72 106.1) (end 155.97 104.85) (width 0.25) (layer F.Cu) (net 8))
 (segment (start 140.65 106.1) (end 154.72 106.1) (width 0.25) (layer F.Cu) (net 8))
 (segment (start 134.6 104.35) (end 136.55 104.35) (width 0.25) (layer F.Cu) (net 9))
 (segment (start 142.6 110.4) (end 142.6 111.35) (width 0.25) (layer F.Cu) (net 9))
 (segment (start 136.55 104.35) (end 142.6 110.4) (width 0.25) (layer F.Cu) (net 9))
 (segment (start 136.05 103.85) (end 136.55 104.35) (width 0.25) (layer F.Cu) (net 9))
 (segment (start 134.6 103.85) (end 136.05 103.85) (width 0.25) (layer F.Cu) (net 9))
 (segment (start 155.97 89.61) (end 157.61 89.61) (width 0.25) (layer B.Cu) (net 10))
 (segment (start 157.61 89.61) (end 158.8 90.8) (width 0.25) (layer B.Cu) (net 10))
 (segment (start 158.8 90.8) (end 158.8 115.15) (width 0.25) (layer B.Cu) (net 10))
 (segment (start 158.8 115.15) (end 157.2 116.75) (width 0.25) (layer B.Cu) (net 10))
 (segment (start 148 116.75) (end 157.2 116.75) (width 0.25) (layer B.Cu) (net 10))
 (segment (start 144.396051 113.146051) (end 148 116.75) (width 0.25) (layer B.Cu) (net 10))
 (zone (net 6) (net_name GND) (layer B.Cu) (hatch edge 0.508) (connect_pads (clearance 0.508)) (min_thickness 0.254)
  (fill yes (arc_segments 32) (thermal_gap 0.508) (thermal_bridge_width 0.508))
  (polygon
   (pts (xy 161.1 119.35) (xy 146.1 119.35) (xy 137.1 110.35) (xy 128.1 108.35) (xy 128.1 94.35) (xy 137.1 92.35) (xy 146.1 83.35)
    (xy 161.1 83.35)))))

